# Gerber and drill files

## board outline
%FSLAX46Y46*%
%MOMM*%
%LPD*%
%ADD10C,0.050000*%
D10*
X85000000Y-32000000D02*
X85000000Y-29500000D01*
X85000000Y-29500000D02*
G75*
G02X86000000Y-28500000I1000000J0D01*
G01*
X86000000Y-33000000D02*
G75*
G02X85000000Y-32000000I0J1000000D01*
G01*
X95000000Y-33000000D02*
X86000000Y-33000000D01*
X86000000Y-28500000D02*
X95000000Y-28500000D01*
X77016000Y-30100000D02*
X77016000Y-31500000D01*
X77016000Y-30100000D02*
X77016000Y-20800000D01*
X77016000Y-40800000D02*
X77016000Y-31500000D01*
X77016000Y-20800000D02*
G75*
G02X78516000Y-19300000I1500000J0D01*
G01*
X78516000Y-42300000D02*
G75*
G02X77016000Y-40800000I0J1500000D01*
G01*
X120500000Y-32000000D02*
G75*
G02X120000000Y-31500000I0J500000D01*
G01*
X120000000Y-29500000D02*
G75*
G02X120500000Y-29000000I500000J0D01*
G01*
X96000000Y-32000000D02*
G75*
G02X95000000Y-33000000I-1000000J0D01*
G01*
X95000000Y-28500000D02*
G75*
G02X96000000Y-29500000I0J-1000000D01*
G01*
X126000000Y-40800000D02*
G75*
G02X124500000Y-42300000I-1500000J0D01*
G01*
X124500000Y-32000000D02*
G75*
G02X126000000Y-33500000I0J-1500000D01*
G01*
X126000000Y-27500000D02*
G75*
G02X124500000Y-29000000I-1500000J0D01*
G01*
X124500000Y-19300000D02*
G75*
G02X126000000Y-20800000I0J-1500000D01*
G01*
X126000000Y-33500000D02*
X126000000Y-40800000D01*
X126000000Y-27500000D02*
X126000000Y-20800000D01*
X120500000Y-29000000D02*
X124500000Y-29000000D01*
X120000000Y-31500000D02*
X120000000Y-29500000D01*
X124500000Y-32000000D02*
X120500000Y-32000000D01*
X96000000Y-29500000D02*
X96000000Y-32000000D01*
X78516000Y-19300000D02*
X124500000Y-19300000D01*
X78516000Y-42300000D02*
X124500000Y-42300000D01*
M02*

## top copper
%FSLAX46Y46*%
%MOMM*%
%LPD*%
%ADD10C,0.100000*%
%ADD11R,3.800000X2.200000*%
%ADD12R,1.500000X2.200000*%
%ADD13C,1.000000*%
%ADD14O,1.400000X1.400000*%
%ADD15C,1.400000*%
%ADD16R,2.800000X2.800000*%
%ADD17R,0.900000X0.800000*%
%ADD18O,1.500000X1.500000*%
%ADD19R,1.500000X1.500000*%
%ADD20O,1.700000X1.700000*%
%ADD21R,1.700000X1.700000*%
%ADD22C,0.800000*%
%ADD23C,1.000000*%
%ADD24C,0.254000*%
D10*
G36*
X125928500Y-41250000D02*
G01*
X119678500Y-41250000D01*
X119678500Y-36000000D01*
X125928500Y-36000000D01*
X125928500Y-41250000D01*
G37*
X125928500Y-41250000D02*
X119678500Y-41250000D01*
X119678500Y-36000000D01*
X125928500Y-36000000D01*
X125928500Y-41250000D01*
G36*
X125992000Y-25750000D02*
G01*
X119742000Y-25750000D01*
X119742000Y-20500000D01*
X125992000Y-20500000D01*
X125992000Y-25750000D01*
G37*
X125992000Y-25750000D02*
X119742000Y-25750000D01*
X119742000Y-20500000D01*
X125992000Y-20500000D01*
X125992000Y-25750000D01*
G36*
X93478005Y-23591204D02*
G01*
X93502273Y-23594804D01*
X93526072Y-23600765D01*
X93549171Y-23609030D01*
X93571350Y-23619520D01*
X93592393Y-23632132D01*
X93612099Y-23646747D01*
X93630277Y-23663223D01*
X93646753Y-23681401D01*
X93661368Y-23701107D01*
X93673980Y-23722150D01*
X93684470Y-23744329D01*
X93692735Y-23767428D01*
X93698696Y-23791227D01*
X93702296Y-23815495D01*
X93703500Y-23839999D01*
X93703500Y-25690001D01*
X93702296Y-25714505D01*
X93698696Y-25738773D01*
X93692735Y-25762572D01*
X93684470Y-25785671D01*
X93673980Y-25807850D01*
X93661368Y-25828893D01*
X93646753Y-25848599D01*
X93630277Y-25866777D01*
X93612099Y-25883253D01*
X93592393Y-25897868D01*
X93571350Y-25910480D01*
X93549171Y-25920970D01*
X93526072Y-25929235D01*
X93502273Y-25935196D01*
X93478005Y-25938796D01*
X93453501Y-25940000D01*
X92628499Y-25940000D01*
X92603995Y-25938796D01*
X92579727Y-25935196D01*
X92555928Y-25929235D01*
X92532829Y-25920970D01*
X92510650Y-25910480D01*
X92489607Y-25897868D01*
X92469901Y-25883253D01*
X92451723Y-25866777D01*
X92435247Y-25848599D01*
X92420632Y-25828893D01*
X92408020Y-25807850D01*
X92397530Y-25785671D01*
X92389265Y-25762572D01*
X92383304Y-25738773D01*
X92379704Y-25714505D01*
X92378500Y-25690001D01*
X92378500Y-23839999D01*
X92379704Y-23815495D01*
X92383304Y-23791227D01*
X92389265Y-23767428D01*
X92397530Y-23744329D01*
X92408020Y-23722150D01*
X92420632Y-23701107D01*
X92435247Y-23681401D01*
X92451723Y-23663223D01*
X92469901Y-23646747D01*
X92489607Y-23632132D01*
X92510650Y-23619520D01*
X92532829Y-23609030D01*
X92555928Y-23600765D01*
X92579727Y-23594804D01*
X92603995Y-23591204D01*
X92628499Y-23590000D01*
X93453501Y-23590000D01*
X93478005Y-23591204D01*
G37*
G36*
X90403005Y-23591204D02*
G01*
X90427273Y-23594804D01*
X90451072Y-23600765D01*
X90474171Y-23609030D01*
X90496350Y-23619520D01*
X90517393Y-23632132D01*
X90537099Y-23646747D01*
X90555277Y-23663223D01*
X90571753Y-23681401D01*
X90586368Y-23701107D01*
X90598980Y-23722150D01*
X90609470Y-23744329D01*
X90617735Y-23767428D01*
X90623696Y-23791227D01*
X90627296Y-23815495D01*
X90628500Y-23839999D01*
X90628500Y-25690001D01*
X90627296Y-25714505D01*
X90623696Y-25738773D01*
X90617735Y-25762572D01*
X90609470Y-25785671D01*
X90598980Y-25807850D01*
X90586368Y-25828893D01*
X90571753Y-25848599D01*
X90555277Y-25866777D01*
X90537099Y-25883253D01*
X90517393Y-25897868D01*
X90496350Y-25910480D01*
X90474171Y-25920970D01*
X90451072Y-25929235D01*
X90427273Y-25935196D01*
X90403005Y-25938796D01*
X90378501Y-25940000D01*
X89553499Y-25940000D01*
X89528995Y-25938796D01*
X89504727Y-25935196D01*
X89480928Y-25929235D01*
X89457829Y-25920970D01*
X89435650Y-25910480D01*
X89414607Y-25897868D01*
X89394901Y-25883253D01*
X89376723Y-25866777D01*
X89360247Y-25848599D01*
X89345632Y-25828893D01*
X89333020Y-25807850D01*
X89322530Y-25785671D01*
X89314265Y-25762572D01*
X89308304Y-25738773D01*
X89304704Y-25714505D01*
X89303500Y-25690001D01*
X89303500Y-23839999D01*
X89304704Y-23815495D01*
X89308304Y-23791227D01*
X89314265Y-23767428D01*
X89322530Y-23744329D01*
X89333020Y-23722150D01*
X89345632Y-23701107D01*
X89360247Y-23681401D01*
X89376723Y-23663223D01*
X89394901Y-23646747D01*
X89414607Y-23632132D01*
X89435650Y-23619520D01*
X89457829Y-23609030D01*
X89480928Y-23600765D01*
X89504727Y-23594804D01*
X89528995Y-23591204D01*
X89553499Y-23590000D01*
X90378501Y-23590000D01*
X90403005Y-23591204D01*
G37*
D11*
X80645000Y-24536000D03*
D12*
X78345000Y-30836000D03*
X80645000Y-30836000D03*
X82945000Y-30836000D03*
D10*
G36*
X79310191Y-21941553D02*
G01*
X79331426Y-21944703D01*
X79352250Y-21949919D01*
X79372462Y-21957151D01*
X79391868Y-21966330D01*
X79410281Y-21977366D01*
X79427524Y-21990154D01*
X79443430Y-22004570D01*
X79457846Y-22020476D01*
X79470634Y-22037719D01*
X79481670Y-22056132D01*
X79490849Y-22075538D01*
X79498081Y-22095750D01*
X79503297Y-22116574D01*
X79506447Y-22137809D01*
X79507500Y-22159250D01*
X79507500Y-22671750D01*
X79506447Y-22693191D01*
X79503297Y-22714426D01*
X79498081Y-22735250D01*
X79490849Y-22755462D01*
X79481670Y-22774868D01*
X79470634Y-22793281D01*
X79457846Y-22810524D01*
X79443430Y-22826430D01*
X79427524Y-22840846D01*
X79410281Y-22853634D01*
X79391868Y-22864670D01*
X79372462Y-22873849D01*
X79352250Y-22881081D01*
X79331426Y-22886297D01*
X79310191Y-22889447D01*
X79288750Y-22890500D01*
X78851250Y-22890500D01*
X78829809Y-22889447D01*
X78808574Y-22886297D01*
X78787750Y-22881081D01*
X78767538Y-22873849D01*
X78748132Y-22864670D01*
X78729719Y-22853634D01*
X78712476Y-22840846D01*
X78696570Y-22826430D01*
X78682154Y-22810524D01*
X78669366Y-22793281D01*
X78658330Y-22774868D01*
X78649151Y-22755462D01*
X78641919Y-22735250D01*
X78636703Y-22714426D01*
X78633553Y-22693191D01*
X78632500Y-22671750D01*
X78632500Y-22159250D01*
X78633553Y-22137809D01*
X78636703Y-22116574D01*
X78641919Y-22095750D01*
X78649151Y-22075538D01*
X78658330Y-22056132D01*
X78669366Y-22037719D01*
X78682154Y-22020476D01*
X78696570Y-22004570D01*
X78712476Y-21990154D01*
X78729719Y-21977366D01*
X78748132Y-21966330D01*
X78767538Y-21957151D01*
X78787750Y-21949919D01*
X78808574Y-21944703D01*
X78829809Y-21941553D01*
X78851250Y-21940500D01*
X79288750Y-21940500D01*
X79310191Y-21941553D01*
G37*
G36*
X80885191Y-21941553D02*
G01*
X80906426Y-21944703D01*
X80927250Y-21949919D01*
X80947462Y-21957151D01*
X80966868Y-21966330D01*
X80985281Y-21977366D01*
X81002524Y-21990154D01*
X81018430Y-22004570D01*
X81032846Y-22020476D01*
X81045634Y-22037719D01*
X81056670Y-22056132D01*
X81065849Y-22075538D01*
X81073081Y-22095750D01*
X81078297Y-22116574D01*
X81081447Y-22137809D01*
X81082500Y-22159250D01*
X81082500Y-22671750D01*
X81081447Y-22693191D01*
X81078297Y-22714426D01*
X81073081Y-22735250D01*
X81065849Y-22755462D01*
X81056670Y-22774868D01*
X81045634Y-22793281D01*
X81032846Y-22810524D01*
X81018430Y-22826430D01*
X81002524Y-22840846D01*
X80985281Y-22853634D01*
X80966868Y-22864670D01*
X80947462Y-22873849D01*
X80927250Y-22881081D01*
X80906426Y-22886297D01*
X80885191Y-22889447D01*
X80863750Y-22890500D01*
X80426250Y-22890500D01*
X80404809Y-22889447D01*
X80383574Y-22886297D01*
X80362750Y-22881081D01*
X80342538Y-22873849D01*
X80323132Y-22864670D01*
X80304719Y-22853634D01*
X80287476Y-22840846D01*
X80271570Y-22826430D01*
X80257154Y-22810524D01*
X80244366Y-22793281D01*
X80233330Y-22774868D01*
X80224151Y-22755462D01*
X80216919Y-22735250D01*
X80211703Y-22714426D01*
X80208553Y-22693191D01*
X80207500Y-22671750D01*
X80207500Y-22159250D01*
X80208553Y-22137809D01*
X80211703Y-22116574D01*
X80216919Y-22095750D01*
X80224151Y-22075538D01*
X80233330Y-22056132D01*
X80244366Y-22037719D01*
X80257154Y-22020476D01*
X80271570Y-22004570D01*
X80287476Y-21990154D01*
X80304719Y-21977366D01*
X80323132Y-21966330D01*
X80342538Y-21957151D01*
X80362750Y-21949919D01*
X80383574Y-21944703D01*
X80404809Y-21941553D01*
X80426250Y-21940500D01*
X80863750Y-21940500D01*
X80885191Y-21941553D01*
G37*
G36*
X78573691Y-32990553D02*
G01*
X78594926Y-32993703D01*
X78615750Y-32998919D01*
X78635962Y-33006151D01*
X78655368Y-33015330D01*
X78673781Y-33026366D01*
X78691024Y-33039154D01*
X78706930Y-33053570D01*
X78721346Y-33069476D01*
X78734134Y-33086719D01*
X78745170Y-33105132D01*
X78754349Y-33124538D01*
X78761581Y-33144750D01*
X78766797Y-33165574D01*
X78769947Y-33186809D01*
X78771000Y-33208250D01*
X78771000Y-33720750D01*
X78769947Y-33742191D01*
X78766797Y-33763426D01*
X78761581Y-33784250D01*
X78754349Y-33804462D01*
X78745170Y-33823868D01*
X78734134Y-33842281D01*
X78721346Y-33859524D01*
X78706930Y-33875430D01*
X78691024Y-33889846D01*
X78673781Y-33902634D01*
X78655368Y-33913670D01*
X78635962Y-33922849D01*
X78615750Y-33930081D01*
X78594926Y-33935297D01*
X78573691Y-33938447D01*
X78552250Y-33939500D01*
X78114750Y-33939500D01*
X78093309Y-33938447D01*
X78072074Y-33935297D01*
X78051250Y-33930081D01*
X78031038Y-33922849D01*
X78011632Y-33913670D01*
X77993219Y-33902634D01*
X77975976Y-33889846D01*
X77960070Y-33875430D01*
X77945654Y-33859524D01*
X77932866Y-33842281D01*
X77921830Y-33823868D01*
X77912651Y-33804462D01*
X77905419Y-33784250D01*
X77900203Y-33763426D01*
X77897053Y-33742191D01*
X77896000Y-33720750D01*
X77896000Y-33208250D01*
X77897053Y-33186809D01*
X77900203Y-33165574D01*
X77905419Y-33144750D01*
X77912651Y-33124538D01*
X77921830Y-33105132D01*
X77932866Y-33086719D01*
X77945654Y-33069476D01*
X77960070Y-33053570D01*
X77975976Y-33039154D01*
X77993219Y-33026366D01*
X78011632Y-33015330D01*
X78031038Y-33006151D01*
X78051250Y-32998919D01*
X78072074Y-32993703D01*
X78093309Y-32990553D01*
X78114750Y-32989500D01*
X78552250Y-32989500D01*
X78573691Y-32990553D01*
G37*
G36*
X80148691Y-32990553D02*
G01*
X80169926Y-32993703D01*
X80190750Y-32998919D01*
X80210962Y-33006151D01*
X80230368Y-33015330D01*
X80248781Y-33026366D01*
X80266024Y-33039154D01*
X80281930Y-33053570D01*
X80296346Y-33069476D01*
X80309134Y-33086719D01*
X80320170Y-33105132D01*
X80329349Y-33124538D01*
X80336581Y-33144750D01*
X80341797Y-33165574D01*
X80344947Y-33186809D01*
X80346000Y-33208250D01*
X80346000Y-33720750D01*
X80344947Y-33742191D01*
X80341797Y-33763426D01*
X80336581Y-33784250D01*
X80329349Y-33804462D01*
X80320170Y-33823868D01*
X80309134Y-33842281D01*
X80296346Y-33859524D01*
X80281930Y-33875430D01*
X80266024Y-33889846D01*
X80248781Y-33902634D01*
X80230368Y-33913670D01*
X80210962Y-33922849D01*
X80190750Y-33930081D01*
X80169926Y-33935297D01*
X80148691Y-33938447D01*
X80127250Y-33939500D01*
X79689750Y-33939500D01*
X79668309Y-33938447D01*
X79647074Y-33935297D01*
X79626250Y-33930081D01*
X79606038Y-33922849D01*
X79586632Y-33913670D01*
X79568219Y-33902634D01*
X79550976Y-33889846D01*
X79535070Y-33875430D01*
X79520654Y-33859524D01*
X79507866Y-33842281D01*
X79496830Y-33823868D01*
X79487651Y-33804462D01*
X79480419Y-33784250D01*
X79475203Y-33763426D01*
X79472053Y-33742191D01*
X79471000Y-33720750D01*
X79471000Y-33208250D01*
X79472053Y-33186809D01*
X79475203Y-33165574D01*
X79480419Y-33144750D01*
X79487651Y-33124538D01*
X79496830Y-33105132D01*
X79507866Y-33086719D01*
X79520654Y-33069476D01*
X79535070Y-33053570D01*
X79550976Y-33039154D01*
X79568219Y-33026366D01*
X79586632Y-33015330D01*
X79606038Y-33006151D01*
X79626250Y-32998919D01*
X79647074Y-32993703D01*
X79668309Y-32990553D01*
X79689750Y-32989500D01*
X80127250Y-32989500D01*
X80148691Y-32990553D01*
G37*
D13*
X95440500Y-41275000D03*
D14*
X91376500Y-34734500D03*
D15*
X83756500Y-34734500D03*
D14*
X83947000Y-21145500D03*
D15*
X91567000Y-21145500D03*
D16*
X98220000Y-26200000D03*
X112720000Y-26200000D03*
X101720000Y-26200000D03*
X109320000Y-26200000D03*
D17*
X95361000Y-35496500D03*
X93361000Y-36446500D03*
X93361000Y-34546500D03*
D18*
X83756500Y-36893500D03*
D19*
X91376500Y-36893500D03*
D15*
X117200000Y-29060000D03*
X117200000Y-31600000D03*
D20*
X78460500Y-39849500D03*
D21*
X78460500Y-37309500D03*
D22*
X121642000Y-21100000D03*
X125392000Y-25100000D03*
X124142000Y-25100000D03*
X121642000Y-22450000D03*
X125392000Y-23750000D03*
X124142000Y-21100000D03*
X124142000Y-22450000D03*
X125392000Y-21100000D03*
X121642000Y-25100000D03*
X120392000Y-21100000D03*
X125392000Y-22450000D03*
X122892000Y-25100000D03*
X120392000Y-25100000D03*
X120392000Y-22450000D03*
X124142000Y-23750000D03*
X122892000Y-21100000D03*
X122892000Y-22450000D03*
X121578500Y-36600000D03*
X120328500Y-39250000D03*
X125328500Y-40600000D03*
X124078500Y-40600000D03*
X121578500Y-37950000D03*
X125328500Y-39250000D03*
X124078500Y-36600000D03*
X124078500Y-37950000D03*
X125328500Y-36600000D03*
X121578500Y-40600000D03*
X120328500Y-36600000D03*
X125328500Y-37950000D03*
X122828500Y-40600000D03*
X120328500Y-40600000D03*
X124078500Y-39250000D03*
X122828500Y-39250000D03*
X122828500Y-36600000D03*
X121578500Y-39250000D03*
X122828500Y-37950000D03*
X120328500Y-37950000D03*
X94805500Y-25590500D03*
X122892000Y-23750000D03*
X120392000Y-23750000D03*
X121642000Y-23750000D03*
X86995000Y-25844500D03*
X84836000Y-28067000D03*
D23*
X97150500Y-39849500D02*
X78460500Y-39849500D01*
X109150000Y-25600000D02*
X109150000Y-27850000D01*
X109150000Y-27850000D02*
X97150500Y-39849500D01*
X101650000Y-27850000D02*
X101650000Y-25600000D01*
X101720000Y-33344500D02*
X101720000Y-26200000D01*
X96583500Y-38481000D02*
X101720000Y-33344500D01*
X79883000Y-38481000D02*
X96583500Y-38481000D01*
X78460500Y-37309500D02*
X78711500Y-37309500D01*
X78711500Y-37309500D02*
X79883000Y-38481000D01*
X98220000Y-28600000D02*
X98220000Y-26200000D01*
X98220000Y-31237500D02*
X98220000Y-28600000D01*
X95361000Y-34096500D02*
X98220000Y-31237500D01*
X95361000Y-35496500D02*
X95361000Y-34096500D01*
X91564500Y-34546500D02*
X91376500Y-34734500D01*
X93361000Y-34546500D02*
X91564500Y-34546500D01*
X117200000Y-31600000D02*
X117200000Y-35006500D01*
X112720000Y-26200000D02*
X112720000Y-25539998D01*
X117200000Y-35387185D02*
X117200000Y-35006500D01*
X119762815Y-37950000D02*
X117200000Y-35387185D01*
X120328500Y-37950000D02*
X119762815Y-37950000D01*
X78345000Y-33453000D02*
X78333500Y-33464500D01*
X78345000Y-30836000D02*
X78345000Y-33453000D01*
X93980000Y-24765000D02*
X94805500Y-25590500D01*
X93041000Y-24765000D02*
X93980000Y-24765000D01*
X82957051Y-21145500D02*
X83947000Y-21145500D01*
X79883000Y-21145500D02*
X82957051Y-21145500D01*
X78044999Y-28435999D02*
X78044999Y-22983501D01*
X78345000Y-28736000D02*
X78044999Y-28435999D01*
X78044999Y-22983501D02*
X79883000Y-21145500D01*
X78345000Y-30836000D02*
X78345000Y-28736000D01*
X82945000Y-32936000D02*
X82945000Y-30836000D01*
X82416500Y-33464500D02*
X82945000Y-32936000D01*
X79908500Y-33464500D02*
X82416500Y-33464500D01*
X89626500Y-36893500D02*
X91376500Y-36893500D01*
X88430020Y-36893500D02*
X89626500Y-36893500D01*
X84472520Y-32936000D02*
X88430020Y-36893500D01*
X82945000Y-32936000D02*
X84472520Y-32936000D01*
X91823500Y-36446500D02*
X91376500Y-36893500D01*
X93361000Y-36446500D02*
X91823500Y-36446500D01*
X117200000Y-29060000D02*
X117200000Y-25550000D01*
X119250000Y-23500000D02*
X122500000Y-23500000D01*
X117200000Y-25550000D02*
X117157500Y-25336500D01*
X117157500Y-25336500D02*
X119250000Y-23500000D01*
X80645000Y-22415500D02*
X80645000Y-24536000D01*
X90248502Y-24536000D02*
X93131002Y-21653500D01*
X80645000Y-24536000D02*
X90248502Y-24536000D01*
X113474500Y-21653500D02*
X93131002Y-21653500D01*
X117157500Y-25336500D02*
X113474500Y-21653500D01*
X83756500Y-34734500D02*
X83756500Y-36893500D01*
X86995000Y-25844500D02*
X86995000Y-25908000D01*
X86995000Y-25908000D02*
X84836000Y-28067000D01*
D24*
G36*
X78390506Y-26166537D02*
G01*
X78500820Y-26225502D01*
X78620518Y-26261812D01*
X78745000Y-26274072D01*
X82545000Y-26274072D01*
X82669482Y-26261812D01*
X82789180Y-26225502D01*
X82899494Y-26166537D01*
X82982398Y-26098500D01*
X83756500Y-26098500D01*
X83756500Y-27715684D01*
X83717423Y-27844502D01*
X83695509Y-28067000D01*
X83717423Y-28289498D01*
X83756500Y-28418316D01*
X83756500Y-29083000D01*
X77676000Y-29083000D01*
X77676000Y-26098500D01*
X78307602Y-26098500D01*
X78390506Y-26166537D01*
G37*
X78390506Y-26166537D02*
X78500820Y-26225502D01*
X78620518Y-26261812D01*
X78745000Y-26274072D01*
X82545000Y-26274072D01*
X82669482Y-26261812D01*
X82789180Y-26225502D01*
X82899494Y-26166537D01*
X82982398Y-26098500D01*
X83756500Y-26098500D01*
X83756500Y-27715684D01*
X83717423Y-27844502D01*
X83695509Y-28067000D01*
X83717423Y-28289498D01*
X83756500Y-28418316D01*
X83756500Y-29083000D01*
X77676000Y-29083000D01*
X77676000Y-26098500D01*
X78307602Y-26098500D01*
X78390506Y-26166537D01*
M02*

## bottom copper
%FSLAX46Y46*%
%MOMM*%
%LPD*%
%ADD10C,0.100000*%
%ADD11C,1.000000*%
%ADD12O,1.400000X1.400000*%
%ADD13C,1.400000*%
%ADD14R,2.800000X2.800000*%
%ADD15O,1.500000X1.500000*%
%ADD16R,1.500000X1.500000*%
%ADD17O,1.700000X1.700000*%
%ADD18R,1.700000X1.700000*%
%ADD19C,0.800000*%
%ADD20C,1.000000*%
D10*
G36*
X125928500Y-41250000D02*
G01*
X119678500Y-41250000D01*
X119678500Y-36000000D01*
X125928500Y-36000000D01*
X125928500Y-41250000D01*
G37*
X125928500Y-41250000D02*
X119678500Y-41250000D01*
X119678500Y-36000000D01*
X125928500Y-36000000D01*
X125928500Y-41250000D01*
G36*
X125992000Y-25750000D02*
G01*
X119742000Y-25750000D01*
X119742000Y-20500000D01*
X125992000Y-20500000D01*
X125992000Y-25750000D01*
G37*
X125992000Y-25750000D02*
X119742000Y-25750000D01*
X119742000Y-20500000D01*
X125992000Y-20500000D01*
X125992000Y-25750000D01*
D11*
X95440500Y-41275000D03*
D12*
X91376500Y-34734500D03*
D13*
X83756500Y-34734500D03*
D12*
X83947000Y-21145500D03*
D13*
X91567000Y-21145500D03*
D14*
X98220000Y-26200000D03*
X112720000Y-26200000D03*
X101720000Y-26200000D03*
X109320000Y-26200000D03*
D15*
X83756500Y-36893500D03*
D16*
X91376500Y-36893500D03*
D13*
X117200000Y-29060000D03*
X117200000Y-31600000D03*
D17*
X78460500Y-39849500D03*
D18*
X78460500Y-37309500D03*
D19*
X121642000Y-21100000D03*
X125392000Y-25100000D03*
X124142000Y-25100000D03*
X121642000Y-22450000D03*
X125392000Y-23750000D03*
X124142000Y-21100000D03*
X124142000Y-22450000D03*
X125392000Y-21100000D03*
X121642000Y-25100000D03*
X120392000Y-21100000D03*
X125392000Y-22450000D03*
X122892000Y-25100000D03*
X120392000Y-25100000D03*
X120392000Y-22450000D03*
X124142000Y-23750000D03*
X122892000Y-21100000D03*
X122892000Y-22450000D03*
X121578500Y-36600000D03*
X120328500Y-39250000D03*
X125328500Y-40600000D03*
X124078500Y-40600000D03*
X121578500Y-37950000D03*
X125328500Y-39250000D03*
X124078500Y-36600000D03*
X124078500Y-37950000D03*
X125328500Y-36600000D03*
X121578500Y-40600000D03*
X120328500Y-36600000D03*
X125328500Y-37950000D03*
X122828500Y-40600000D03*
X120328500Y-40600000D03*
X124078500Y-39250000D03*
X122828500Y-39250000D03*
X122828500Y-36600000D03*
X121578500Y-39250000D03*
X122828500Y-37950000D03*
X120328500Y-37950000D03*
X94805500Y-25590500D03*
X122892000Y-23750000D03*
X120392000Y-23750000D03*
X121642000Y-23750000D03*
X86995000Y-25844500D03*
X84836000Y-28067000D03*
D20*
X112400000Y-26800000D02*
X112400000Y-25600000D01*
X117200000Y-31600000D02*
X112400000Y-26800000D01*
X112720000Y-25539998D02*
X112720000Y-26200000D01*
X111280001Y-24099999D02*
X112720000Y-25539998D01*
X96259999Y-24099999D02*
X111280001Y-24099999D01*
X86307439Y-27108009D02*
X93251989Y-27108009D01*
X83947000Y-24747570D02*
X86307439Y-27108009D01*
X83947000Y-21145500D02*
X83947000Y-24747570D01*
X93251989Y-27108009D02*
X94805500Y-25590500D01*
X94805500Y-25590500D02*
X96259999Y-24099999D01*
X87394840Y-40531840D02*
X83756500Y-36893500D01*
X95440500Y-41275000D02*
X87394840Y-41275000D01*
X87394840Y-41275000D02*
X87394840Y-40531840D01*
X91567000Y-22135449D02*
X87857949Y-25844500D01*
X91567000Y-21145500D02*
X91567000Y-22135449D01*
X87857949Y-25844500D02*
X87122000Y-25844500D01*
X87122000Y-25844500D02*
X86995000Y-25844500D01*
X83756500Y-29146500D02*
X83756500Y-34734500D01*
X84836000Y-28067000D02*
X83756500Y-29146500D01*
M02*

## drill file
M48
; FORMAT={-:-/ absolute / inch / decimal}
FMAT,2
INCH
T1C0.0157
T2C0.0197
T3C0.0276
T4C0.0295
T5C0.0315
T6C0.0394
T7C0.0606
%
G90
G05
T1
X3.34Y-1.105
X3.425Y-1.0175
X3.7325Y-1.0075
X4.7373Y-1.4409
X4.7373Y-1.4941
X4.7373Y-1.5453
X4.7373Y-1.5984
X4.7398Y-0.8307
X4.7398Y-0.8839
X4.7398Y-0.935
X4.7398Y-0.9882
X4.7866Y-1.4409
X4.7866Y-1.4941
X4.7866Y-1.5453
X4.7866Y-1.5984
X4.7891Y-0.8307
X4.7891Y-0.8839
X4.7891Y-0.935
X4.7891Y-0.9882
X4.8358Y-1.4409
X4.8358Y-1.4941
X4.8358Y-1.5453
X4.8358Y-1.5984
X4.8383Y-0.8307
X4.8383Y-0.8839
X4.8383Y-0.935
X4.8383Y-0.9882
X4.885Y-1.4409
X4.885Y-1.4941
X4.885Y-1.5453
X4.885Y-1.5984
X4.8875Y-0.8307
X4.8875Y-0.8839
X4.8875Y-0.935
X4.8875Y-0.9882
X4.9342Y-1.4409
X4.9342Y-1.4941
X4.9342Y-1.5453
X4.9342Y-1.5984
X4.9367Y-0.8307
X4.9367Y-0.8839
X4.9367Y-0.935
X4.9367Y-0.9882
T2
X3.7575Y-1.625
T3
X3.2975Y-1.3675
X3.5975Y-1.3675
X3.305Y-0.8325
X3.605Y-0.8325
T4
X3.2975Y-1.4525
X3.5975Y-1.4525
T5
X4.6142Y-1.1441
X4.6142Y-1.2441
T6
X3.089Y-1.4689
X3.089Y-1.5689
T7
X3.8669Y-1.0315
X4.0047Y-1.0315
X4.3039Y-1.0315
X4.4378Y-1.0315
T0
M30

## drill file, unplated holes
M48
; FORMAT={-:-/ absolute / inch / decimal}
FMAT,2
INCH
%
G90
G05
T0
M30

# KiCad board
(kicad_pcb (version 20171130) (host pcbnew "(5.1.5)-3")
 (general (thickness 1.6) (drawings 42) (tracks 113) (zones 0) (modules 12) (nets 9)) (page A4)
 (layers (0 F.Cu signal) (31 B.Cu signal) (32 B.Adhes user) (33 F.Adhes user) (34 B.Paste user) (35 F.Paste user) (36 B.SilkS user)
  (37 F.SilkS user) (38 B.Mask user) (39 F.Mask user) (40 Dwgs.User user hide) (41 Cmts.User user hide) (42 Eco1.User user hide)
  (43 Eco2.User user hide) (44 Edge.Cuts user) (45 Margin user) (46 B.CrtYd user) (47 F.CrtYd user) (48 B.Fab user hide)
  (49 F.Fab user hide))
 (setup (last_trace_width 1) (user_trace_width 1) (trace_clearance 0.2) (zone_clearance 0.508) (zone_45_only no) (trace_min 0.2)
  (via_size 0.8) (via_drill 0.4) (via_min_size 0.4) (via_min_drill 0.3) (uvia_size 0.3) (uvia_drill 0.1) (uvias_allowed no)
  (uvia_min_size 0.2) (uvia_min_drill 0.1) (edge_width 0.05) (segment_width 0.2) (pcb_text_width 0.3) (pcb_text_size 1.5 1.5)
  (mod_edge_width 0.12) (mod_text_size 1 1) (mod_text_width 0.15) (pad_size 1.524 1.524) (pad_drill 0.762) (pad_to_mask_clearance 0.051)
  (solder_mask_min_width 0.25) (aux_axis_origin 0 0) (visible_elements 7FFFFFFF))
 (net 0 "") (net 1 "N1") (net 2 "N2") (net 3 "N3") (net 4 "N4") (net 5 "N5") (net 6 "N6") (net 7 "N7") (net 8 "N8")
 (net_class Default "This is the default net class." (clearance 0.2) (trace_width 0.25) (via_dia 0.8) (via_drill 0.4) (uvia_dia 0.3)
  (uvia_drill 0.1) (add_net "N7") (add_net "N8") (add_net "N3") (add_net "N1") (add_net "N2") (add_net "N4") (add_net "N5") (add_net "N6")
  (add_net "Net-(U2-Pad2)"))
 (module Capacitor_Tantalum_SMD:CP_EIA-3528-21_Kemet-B (layer F.Cu) (at 91.5035 24.765)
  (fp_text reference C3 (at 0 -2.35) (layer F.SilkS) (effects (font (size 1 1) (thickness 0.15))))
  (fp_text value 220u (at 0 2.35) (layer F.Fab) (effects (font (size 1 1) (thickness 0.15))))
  (pad 2 smd roundrect (at 1.5375 0) (size 1.325 2.35) (layers F.Cu F.Paste F.Mask) (roundrect_rratio 0.188679) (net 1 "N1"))
  (pad 1 smd roundrect (at -1.5375 0) (size 1.325 2.35) (layers F.Cu F.Paste F.Mask) (roundrect_rratio 0.188679) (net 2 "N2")))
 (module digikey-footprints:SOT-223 (layer F.Cu) (at 80.645 27.686)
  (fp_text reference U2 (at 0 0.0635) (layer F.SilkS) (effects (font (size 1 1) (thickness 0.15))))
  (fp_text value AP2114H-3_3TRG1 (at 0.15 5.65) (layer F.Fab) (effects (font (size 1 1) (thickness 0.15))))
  (pad 4 smd rect (at 0 -3.15) (size 3.8 2.2) (layers F.Cu F.Paste F.Mask) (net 2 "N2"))
  (pad 1 smd rect (at -2.3 3.15) (size 1.5 2.2) (layers F.Cu F.Paste F.Mask) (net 1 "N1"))
  (pad 2 smd rect (at 0 3.15) (size 1.5 2.2) (layers F.Cu F.Paste F.Mask))
  (pad 3 smd rect (at 2.3 3.15) (size 1.5 2.2) (layers F.Cu F.Paste F.Mask) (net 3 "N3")))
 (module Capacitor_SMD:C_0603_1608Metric (layer F.Cu) (at 79.8575 22.4155 180)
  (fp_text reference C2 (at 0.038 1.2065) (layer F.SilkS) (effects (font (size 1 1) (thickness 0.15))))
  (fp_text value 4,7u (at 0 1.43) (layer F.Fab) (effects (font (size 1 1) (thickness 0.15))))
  (pad 2 smd roundrect (at 0.7875 0 180) (size 0.875 0.95) (layers F.Cu F.Paste F.Mask) (roundrect_rratio 0.25) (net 1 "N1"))
  (pad 1 smd roundrect (at -0.7875 0 180) (size 0.875 0.95) (layers F.Cu F.Paste F.Mask) (roundrect_rratio 0.25) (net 2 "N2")))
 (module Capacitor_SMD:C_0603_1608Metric (layer F.Cu) (at 79.121 33.4645 180)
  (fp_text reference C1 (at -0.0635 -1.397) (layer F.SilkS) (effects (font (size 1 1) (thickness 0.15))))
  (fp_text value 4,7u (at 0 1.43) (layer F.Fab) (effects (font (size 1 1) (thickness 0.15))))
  (pad 2 smd roundrect (at 0.7875 0 180) (size 0.875 0.95) (layers F.Cu F.Paste F.Mask) (roundrect_rratio 0.25) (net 1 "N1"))
  (pad 1 smd roundrect (at -0.7875 0 180) (size 0.875 0.95) (layers F.Cu F.Paste F.Mask) (roundrect_rratio 0.25) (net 3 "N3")))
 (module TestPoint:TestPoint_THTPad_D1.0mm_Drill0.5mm (layer F.Cu) (at 95.4405 41.275)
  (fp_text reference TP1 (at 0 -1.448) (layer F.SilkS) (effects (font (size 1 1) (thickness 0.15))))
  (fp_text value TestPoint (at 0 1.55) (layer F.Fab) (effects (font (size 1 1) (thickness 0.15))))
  (pad 1 thru_hole circle (at 0 0) (size 1 1) (drill 0.5) (layers *.Cu *.Mask) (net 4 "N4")))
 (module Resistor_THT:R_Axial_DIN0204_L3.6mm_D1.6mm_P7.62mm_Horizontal (layer F.Cu) (at 83.7565 34.7345)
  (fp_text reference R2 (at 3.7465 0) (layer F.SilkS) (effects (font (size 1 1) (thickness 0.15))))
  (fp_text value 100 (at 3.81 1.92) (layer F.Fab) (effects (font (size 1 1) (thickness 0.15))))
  (pad 2 thru_hole oval (at 7.62 0) (size 1.4 1.4) (drill 0.7) (layers *.Cu *.Mask) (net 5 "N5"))
  (pad 1 thru_hole circle (at 0 0) (size 1.4 1.4) (drill 0.7) (layers *.Cu *.Mask) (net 4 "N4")))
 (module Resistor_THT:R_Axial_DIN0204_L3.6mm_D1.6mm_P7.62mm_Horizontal (layer F.Cu) (at 91.567 21.1455 180)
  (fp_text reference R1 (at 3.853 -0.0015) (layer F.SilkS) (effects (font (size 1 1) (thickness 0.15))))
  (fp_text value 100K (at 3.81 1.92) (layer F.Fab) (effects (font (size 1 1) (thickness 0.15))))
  (pad 2 thru_hole oval (at 7.62 0 180) (size 1.4 1.4) (drill 0.7) (layers *.Cu *.Mask) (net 1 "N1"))
  (pad 1 thru_hole circle (at 0 0 180) (size 1.4 1.4) (drill 0.7) (layers *.Cu *.Mask) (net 4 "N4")))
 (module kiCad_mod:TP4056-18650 (layer F.Cu) (at 96.52 50.8 90)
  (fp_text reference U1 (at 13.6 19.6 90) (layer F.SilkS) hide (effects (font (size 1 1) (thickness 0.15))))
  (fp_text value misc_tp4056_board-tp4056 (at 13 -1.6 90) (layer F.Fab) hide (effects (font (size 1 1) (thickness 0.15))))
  (pad 5 thru_hole rect (at 24.6 1.7 90) (size 2.8 2.8) (drill 1.54) (layers *.Cu *.Mask) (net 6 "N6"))
  (pad 6 thru_hole rect (at 24.6 16.2 90) (size 2.8 2.8) (drill 1.54) (layers *.Cu *.Mask) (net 1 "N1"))
  (pad 3 thru_hole rect (at 24.6 5.2 90) (size 2.8 2.8) (drill 1.54) (layers *.Cu *.Mask) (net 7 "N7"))
  (pad 4 thru_hole rect (at 24.6 12.8 90) (size 2.8 2.8) (drill 1.54) (layers *.Cu *.Mask) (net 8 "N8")))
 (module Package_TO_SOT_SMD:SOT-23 (layer F.Cu) (at 94.361 35.4965)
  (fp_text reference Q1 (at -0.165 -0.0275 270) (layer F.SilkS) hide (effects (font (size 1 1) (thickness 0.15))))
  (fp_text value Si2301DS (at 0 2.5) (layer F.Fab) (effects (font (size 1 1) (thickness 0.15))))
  (pad 3 smd rect (at 1 0) (size 0.9 0.8) (layers F.Cu F.Paste F.Mask) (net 6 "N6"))
  (pad 2 smd rect (at -1 0.95) (size 0.9 0.8) (layers F.Cu F.Paste F.Mask) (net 3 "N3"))
  (pad 1 smd rect (at -1 -0.95) (size 0.9 0.8) (layers F.Cu F.Paste F.Mask) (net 5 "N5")))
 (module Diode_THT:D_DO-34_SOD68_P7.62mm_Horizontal (layer F.Cu) (at 91.3765 36.8935 180)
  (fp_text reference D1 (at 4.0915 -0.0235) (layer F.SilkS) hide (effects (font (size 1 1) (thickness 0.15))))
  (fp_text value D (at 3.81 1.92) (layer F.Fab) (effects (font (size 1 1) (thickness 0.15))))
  (pad 2 thru_hole oval (at 7.62 0 180) (size 1.5 1.5) (drill 0.75) (layers *.Cu *.Mask) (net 4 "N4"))
  (pad 1 thru_hole rect (at 0 0 180) (size 1.5 1.5) (drill 0.75) (layers *.Cu *.Mask) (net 3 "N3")))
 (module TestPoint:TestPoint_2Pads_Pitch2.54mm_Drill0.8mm (layer F.Cu) (at 117.2 31.6 90)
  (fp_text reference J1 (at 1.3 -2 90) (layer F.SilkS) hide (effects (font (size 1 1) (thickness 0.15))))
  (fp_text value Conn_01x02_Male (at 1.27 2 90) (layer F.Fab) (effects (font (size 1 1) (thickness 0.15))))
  (pad 2 thru_hole circle (at 2.54 0 90) (size 1.4 1.4) (drill 0.8) (layers *.Cu *.Mask) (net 2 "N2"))
  (pad 1 thru_hole circle (at 0 0 90) (size 1.4 1.4) (drill 0.8) (layers *.Cu *.Mask) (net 1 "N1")))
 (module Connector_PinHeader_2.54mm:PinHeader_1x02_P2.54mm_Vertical (layer F.Cu) (at 78.4605 37.3095)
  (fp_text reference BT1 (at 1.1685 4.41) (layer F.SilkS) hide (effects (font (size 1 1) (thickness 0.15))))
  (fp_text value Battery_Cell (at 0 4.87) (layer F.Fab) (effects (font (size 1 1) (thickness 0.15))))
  (pad 2 thru_hole oval (at 0 2.54) (size 1.7 1.7) (drill 1) (layers *.Cu *.Mask) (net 8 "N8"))
  (pad 1 thru_hole rect (at 0 0) (size 1.7 1.7) (drill 1) (layers *.Cu *.Mask) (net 7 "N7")))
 (gr_line (start 85 32) (end 85 29.5) (layer Edge.Cuts) (width 0.05))
 (gr_arc (start 86 29.5) (end 86 28.5) (angle -90) (layer Edge.Cuts) (width 0.05))
 (gr_arc (start 86 32) (end 85 32) (angle -90) (layer Edge.Cuts) (width 0.05))
 (gr_line (start 95 33) (end 86 33) (layer Edge.Cuts) (width 0.05))
 (gr_line (start 86 28.5) (end 95 28.5) (layer Edge.Cuts) (width 0.05))
 (gr_line (start 77.016 30.1) (end 77.016 31.5) (layer Edge.Cuts) (width 0.05))
 (gr_line (start 77.016 30.1) (end 77.016 20.8) (layer Edge.Cuts) (width 0.05))
 (gr_line (start 77.016 40.8) (end 77.016 31.5) (layer Edge.Cuts) (width 0.05))
 (gr_arc (start 78.516 20.8) (end 78.516 19.3) (angle -90) (layer Edge.Cuts) (width 0.05))
 (gr_arc (start 78.516 40.8) (end 77.016 40.8) (angle -90) (layer Edge.Cuts) (width 0.05))
 (gr_poly (pts (xy 125.9285 41.25) (xy 119.6785 41.25) (xy 119.6785 36) (xy 125.9285 36)) (layer B.Cu) (width 0.1))
 (gr_poly (pts (xy 125.9285 41.25) (xy 119.6785 41.25) (xy 119.6785 36) (xy 125.9285 36)) (layer F.Cu) (width 0.1))
 (gr_poly (pts (xy 125.992 25.75) (xy 119.742 25.75) (xy 119.742 20.5) (xy 125.992 20.5)) (layer B.Cu) (width 0.1))
 (gr_arc (start 120.5 31.5) (end 120 31.5) (angle -90) (layer Edge.Cuts) (width 0.05))
 (gr_arc (start 120.5 29.5) (end 120.5 29) (angle -90) (layer Edge.Cuts) (width 0.05))
 (gr_poly (pts (xy 125.992 25.75) (xy 119.742 25.75) (xy 119.742 20.5) (xy 125.992 20.5)) (layer F.Cu) (width 0.1))
 (gr_arc (start 95 32) (end 95 33) (angle -90) (layer Edge.Cuts) (width 0.05))
 (gr_arc (start 95 29.5) (end 96 29.5) (angle -90) (layer Edge.Cuts) (width 0.05))
 (gr_arc (start 124.5 40.8) (end 124.5 42.3) (angle -90) (layer Edge.Cuts) (width 0.05))
 (gr_arc (start 124.5 33.5) (end 126 33.5) (angle -90) (layer Edge.Cuts) (width 0.05))
 (gr_arc (start 124.5 27.5) (end 124.5 29) (angle -90) (layer Edge.Cuts) (width 0.05))
 (gr_arc (start 124.5 20.8) (end 126 20.8) (angle -90) (layer Edge.Cuts) (width 0.05))
 (gr_line (start 126 33.5) (end 126 40.8) (layer Edge.Cuts) (width 0.05))
 (gr_line (start 126 27.5) (end 126 20.8) (layer Edge.Cuts) (width 0.05))
 (gr_line (start 120.5 29) (end 124.5 29) (layer Edge.Cuts) (width 0.05))
 (gr_line (start 120 31.5) (end 120 29.5) (layer Edge.Cuts) (width 0.05))
 (gr_line (start 124.5 32) (end 120.5 32) (layer Edge.Cuts) (width 0.05))
 (gr_line (start 96 29.5) (end 96 32) (layer Edge.Cuts) (width 0.05))
 (gr_line (start 78.516 19.3) (end 124.5 19.3) (layer Edge.Cuts) (width 0.05))
 (gr_line (start 78.516 42.3) (end 124.5 42.3) (layer Edge.Cuts) (width 0.05))
 (via (at 121.642 21.1) (size 0.8) (drill 0.4) (layers F.Cu B.Cu) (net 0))
 (via (at 125.392 25.1) (size 0.8) (drill 0.4) (layers F.Cu B.Cu) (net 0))
 (via (at 124.142 25.1) (size 0.8) (drill 0.4) (layers F.Cu B.Cu) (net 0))
 (via (at 121.642 22.45) (size 0.8) (drill 0.4) (layers F.Cu B.Cu) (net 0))
 (via (at 125.392 23.75) (size 0.8) (drill 0.4) (layers F.Cu B.Cu) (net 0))
 (via (at 124.142 21.1) (size 0.8) (drill 0.4) (layers F.Cu B.Cu) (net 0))
 (via (at 124.142 22.45) (size 0.8) (drill 0.4) (layers F.Cu B.Cu) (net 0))
 (via (at 125.392 21.1) (size 0.8) (drill 0.4) (layers F.Cu B.Cu) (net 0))
 (via (at 121.642 25.1) (size 0.8) (drill 0.4) (layers F.Cu B.Cu) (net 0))
 (via (at 120.392 21.1) (size 0.8) (drill 0.4) (layers F.Cu B.Cu) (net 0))
 (via (at 125.392 22.45) (size 0.8) (drill 0.4) (layers F.Cu B.Cu) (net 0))
 (via (at 122.892 25.1) (size 0.8) (drill 0.4) (layers F.Cu B.Cu) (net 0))
 (via (at 120.392 25.1) (size 0.8) (drill 0.4) (layers F.Cu B.Cu) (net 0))
 (via (at 120.392 22.45) (size 0.8) (drill 0.4) (layers F.Cu B.Cu) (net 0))
 (via (at 124.142 23.75) (size 0.8) (drill 0.4) (layers F.Cu B.Cu) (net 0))
 (via (at 122.892 21.1) (size 0.8) (drill 0.4) (layers F.Cu B.Cu) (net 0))
 (via (at 122.892 22.45) (size 0.8) (drill 0.4) (layers F.Cu B.Cu) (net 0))
 (via (at 121.5785 36.6) (size 0.8) (drill 0.4) (layers F.Cu B.Cu) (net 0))
 (via (at 120.3285 39.25) (size 0.8) (drill 0.4) (layers F.Cu B.Cu) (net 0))
 (via (at 125.3285 40.6) (size 0.8) (drill 0.4) (layers F.Cu B.Cu) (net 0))
 (via (at 124.0785 40.6) (size 0.8) (drill 0.4) (layers F.Cu B.Cu) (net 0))
 (via (at 121.5785 37.95) (size 0.8) (drill 0.4) (layers F.Cu B.Cu) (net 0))
 (via (at 125.3285 39.25) (size 0.8) (drill 0.4) (layers F.Cu B.Cu) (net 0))
 (via (at 124.0785 36.6) (size 0.8) (drill 0.4) (layers F.Cu B.Cu) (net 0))
 (via (at 124.0785 37.95) (size 0.8) (drill 0.4) (layers F.Cu B.Cu) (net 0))
 (via (at 125.3285 36.6) (size 0.8) (drill 0.4) (layers F.Cu B.Cu) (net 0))
 (via (at 121.5785 40.6) (size 0.8) (drill 0.4) (layers F.Cu B.Cu) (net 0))
 (via (at 120.3285 36.6) (size 0.8) (drill 0.4) (layers F.Cu B.Cu) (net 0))
 (via (at 125.3285 37.95) (size 0.8) (drill 0.4) (layers F.Cu B.Cu) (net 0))
 (via (at 122.8285 40.6) (size 0.8) (drill 0.4) (layers F.Cu B.Cu) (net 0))
 (via (at 120.3285 40.6) (size 0.8) (drill 0.4) (layers F.Cu B.Cu) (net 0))
 (via (at 124.0785 39.25) (size 0.8) (drill 0.4) (layers F.Cu B.Cu) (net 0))
 (via (at 122.8285 39.25) (size 0.8) (drill 0.4) (layers F.Cu B.Cu) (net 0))
 (via (at 122.8285 36.6) (size 0.8) (drill 0.4) (layers F.Cu B.Cu) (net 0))
 (via (at 121.5785 39.25) (size 0.8) (drill 0.4) (layers F.Cu B.Cu) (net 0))
 (via (at 122.8285 37.95) (size 0.8) (drill 0.4) (layers F.Cu B.Cu) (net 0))
 (segment (start 97.1505 39.8495) (end 78.4605 39.8495) (width 1) (layer F.Cu) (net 8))
 (segment (start 109.15 25.6) (end 109.15 27.85) (width 1) (layer F.Cu) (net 8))
 (segment (start 109.15 27.85) (end 97.1505 39.8495) (width 1) (layer F.Cu) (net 8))
 (segment (start 101.65 27.85) (end 101.65 25.6) (width 1) (layer F.Cu) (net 7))
 (segment (start 101.72 33.3445) (end 101.72 26.2) (width 1) (layer F.Cu) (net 7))
 (segment (start 96.5835 38.481) (end 101.72 33.3445) (width 1) (layer F.Cu) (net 7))
 (segment (start 79.883 38.481) (end 96.5835 38.481) (width 1) (layer F.Cu) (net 7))
 (segment (start 78.4605 37.3095) (end 78.7115 37.3095) (width 1) (layer F.Cu) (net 7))
 (segment (start 78.7115 37.3095) (end 79.883 38.481) (width 1) (layer F.Cu) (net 7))
 (segment (start 98.22 28.6) (end 98.22 26.2) (width 1) (layer F.Cu) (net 6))
 (segment (start 98.22 31.2375) (end 98.22 28.6) (width 1) (layer F.Cu) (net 6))
 (segment (start 95.361 34.0965) (end 98.22 31.2375) (width 1) (layer F.Cu) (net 6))
 (segment (start 95.361 35.4965) (end 95.361 34.0965) (width 1) (layer F.Cu) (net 6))
 (segment (start 91.5645 34.5465) (end 91.3765 34.7345) (width 1) (layer F.Cu) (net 5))
 (segment (start 93.361 34.5465) (end 91.5645 34.5465) (width 1) (layer F.Cu) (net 5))
 (segment (start 112.4 26.8) (end 112.4 25.6) (width 1) (layer B.Cu) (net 1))
 (segment (start 117.2 31.6) (end 112.4 26.8) (width 1) (layer B.Cu) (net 1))
 (segment (start 117.2 31.6) (end 117.2 35.0065) (width 1) (layer F.Cu) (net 1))
 (segment (start 112.72 26.2) (end 112.72 25.539998) (width 1) (layer F.Cu) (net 1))
 (via (at 120.3285 37.95) (size 0.8) (drill 0.4) (layers F.Cu B.Cu) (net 1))
 (segment (start 117.2 35.387185) (end 117.2 35.0065) (width 1) (layer F.Cu) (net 1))
 (segment (start 119.762815 37.95) (end 117.2 35.387185) (width 1) (layer F.Cu) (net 1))
 (segment (start 120.3285 37.95) (end 119.762815 37.95) (width 1) (layer F.Cu) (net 1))
 (segment (start 78.345 33.453) (end 78.3335 33.4645) (width 1) (layer F.Cu) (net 1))
 (segment (start 78.345 30.836) (end 78.345 33.453) (width 1) (layer F.Cu) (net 1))
 (segment (start 112.72 25.539998) (end 112.72 26.2) (width 1) (layer B.Cu) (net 1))
 (segment (start 111.280001 24.099999) (end 112.72 25.539998) (width 1) (layer B.Cu) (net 1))
 (segment (start 96.259999 24.099999) (end 111.280001 24.099999) (width 1) (layer B.Cu) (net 1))
 (segment (start 86.307439 27.108009) (end 93.251989 27.108009) (width 1) (layer B.Cu) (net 1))
 (segment (start 83.947 24.74757) (end 86.307439 27.108009) (width 1) (layer B.Cu) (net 1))
 (segment (start 83.947 21.1455) (end 83.947 24.74757) (width 1) (layer B.Cu) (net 1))
 (via (at 94.8055 25.5905) (size 0.8) (drill 0.4) (layers F.Cu B.Cu) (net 1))
 (segment (start 93.98 24.765) (end 94.8055 25.5905) (width 1) (layer F.Cu) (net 1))
 (segment (start 93.041 24.765) (end 93.98 24.765) (width 1) (layer F.Cu) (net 1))
 (segment (start 93.251989 27.108009) (end 94.8055 25.5905) (width 1) (layer B.Cu) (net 1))
 (segment (start 94.8055 25.5905) (end 96.259999 24.099999) (width 1) (layer B.Cu) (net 1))
 (segment (start 82.957051 21.1455) (end 83.947 21.1455) (width 1) (layer F.Cu) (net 1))
 (segment (start 79.883 21.1455) (end 82.957051 21.1455) (width 1) (layer F.Cu) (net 1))
 (segment (start 78.044999 28.435999) (end 78.044999 22.983501) (width 1) (layer F.Cu) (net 1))
 (segment (start 78.345 28.736) (end 78.044999 28.435999) (width 1) (layer F.Cu) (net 1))
 (segment (start 78.044999 22.983501) (end 79.883 21.1455) (width 1) (layer F.Cu) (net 1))
 (segment (start 78.345 30.836) (end 78.345 28.736) (width 1) (layer F.Cu) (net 1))
 (segment (start 82.945 32.936) (end 82.945 30.836) (width 1) (layer F.Cu) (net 3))
 (segment (start 82.4165 33.4645) (end 82.945 32.936) (width 1) (layer F.Cu) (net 3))
 (segment (start 79.9085 33.4645) (end 82.4165 33.4645) (width 1) (layer F.Cu) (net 3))
 (segment (start 89.6265 36.8935) (end 91.3765 36.8935) (width 1) (layer F.Cu) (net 3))
 (segment (start 88.43002 36.8935) (end 89.6265 36.8935) (width 1) (layer F.Cu) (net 3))
 (segment (start 84.47252 32.936) (end 88.43002 36.8935) (width 1) (layer F.Cu) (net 3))
 (segment (start 82.945 32.936) (end 84.47252 32.936) (width 1) (layer F.Cu) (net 3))
 (segment (start 91.8235 36.4465) (end 91.3765 36.8935) (width 1) (layer F.Cu) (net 3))
 (segment (start 93.361 36.4465) (end 91.8235 36.4465) (width 1) (layer F.Cu) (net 3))
 (via (at 122.892 23.75) (size 0.8) (drill 0.4) (layers F.Cu B.Cu) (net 2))
 (via (at 120.392 23.75) (size 0.8) (drill 0.4) (layers F.Cu B.Cu) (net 2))
 (via (at 121.642 23.75) (size 0.8) (drill 0.4) (layers F.Cu B.Cu) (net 2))
 (segment (start 117.2 29.06) (end 117.2 25.55) (width 1) (layer F.Cu) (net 2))
 (segment (start 119.25 23.5) (end 122.5 23.5) (width 1) (layer F.Cu) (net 2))
 (segment (start 117.2 25.55) (end 117.1575 25.3365) (width 1) (layer F.Cu) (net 2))
 (segment (start 117.1575 25.3365) (end 119.25 23.5) (width 1) (layer F.Cu) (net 2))
 (segment (start 80.645 22.4155) (end 80.645 24.536) (width 1) (layer F.Cu) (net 2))
 (segment (start 90.248502 24.536) (end 93.131002 21.6535) (width 1) (layer F.Cu) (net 2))
 (segment (start 80.645 24.536) (end 90.248502 24.536) (width 1) (layer F.Cu) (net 2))
 (segment (start 113.4745 21.6535) (end 93.131002 21.6535) (width 1) (layer F.Cu) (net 2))
 (segment (start 117.1575 25.3365) (end 113.4745 21.6535) (width 1) (layer F.Cu) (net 2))
 (segment (start 87.39484 40.53184) (end 83.7565 36.8935) (width 1) (layer B.Cu) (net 4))
 (segment (start 95.4405 41.275) (end 87.39484 41.275) (width 1) (layer B.Cu) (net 4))
 (segment (start 87.39484 41.275) (end 87.39484 40.53184) (width 1) (layer B.Cu) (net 4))
 (segment (start 83.7565 34.7345) (end 83.7565 36.8935) (width 1) (layer F.Cu) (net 4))
 (segment (start 91.567 22.135449) (end 87.857949 25.8445) (width 1) (layer B.Cu) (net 4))
 (segment (start 91.567 21.1455) (end 91.567 22.135449) (width 1) (layer B.Cu) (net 4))
 (via (at 86.995 25.8445) (size 0.8) (drill 0.4) (layers F.Cu B.Cu) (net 4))
 (segment (start 87.857949 25.8445) (end 87.122 25.8445) (width 1) (layer B.Cu) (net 4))
 (segment (start 87.122 25.8445) (end 86.995 25.8445) (width 1) (layer B.Cu) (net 4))
 (via (at 84.836 28.067) (size 0.8) (drill 0.4) (layers F.Cu B.Cu) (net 4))
 (segment (start 86.995 25.8445) (end 86.995 25.908) (width 1) (layer F.Cu) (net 4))
 (segment (start 86.995 25.908) (end 84.836 28.067) (width 1) (layer F.Cu) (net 4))
 (segment (start 83.7565 29.1465) (end 83.7565 34.7345) (width 1) (layer B.Cu) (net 4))
 (segment (start 84.836 28.067) (end 83.7565 29.1465) (width 1) (layer B.Cu) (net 4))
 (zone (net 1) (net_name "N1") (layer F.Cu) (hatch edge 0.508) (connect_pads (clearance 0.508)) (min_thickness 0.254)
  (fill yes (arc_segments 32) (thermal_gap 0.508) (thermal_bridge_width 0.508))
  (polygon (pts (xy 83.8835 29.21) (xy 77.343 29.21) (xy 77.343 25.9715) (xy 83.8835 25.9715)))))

